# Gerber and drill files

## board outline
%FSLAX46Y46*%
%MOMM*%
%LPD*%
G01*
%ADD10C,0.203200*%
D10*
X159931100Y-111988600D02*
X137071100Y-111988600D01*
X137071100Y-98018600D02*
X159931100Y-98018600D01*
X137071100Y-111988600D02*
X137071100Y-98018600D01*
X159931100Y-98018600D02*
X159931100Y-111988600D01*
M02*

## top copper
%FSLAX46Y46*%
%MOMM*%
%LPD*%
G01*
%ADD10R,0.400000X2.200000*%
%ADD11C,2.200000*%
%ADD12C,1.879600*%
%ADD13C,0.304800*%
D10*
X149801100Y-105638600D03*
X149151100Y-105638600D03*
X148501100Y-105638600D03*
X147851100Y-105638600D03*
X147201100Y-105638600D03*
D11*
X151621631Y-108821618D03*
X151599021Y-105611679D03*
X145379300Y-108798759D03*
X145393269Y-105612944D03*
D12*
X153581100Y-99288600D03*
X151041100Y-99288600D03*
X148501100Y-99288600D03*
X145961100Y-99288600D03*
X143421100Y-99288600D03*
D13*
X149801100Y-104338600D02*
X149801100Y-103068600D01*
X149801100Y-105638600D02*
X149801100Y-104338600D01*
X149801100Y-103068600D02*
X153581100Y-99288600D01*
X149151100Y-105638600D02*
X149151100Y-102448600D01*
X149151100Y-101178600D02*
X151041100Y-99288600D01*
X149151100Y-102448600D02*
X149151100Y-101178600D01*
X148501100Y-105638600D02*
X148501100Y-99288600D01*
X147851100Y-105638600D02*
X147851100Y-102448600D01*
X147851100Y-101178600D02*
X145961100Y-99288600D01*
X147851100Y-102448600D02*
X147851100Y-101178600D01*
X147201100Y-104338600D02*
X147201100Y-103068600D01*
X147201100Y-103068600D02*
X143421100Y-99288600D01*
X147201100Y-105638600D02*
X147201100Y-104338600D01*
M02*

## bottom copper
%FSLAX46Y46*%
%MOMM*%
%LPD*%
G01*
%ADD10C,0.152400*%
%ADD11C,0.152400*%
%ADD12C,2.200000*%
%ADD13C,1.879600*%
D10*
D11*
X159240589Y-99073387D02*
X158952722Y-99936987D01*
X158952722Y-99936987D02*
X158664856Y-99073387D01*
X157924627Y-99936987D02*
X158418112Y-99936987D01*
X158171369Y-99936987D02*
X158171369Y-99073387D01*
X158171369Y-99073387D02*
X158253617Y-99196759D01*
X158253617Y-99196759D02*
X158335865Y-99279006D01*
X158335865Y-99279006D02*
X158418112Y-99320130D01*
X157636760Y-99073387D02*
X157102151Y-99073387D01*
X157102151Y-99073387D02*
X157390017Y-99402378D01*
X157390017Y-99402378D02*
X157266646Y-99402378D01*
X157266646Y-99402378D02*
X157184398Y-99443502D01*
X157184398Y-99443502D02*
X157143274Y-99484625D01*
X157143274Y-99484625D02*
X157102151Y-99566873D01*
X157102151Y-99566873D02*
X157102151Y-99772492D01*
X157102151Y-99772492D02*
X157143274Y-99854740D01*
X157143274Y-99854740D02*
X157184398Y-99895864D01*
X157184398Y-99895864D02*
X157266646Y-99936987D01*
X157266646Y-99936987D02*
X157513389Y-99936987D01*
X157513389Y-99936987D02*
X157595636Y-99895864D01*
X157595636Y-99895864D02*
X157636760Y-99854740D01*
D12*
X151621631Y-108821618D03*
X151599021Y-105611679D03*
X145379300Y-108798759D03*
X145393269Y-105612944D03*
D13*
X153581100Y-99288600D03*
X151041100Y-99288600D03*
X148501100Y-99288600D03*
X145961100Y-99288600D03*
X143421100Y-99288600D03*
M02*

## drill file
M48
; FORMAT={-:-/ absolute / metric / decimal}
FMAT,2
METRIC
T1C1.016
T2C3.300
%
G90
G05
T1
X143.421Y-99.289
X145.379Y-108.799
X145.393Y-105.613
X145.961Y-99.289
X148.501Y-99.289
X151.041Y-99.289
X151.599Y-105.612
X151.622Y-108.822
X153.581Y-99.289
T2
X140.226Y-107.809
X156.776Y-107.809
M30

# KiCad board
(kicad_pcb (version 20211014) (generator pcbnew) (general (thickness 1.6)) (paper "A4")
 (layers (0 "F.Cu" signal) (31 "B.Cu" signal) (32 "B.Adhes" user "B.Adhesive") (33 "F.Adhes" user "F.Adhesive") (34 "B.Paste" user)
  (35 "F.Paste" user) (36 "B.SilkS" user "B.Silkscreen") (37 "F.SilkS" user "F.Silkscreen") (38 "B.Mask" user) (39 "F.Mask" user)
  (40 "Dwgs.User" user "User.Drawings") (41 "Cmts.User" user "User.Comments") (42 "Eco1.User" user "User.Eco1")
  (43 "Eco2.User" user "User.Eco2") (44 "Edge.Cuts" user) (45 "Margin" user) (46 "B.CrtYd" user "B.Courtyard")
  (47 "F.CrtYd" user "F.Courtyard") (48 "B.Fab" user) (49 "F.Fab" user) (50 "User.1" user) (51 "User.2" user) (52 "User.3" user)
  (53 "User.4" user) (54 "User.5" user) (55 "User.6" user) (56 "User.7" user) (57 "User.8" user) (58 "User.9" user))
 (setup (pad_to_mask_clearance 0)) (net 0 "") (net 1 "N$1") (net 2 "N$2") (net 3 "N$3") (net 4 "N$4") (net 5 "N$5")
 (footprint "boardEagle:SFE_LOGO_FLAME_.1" (layer "F.Cu") (at 156.7561 101.3206)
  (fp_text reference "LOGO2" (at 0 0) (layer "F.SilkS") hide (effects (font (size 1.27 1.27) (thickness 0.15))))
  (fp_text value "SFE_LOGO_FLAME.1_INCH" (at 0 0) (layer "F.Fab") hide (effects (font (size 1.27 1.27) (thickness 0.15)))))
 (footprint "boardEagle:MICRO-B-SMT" (layer "F.Cu") (at 148.5011 105.6386 180)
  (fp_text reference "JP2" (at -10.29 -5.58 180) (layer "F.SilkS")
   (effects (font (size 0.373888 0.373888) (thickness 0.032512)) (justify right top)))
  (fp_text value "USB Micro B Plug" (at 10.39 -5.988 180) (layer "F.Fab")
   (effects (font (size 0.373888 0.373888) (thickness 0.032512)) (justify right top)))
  (pad "" np_thru_hole circle (at -8.275 -2.17 180) (size 3.3 3.3) (drill 3.3) (layers *.Cu *.Mask))
  (pad "" np_thru_hole circle (at 8.275 -2.17 180) (size 3.3 3.3) (drill 3.3) (layers *.Cu *.Mask))
  (pad "1" smd rect (at -1.3 0 270) (size 2.2 0.4) (layers "F.Cu" "F.Paste" "F.Mask") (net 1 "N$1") (solder_mask_margin 0.1016))
  (pad "2" smd rect (at -0.65 0 270) (size 2.2 0.4) (layers "F.Cu" "F.Paste" "F.Mask") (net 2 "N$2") (solder_mask_margin 0.1016))
  (pad "3" smd rect (at 0 0 270) (size 2.2 0.4) (layers "F.Cu" "F.Paste" "F.Mask") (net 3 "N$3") (solder_mask_margin 0.1016))
  (pad "4" smd rect (at 0.65 0 270) (size 2.2 0.4) (layers "F.Cu" "F.Paste" "F.Mask") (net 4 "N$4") (solder_mask_margin 0.1016))
  (pad "5" smd rect (at 1.3 0 270) (size 2.2 0.4) (layers "F.Cu" "F.Paste" "F.Mask") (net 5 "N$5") (solder_mask_margin 0.1016))
  (pad "P$6" thru_hole circle (at -3.120531 -3.183018 270) (size 2.2 2.2) (drill 1.016) (layers *.Cu *.Mask) (solder_mask_margin 0.1016))
  (pad "P$7" thru_hole circle (at -3.097921 0.026921 270) (size 2.2 2.2) (drill 1.016) (layers *.Cu *.Mask) (solder_mask_margin 0.1016))
  (pad "P$8" thru_hole circle (at 3.1218 -3.160159 270) (size 2.2 2.2) (drill 1.016) (layers *.Cu *.Mask) (solder_mask_margin 0.1016))
  (pad "P$9" thru_hole circle (at 3.107831 0.025656 270) (size 2.2 2.2) (drill 1.016) (layers *.Cu *.Mask) (solder_mask_margin 0.1016)))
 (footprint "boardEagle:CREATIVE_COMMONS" (layer "F.Cu") (at 121.707044 124.1806)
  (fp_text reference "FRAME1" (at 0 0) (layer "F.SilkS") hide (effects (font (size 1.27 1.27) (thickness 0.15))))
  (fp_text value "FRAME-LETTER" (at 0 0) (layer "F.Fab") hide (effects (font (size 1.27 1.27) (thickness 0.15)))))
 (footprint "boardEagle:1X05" (layer "F.Cu") (at 153.5811 99.2886 180)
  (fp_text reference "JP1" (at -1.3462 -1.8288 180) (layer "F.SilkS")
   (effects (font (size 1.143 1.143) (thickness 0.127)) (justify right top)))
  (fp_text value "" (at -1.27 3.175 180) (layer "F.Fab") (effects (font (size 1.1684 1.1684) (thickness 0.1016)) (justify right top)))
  (pad "1" thru_hole circle (at 0 0 270) (size 1.8796 1.8796) (drill 1.016) (layers *.Cu *.Mask) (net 1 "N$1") (solder_mask_margin 0.1016))
  (pad "2" thru_hole circle (at 2.54 0 270) (size 1.8796 1.8796) (drill 1.016) (layers *.Cu *.Mask) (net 2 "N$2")
   (solder_mask_margin 0.1016))
  (pad "3" thru_hole circle (at 5.08 0 270) (size 1.8796 1.8796) (drill 1.016) (layers *.Cu *.Mask) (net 3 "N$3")
   (solder_mask_margin 0.1016))
  (pad "4" thru_hole circle (at 7.62 0 270) (size 1.8796 1.8796) (drill 1.016) (layers *.Cu *.Mask) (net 4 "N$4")
   (solder_mask_margin 0.1016))
  (pad "5" thru_hole circle (at 10.16 0 270) (size 1.8796 1.8796) (drill 1.016) (layers *.Cu *.Mask) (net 5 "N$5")
   (solder_mask_margin 0.1016)))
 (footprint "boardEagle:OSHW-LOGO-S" (layer "F.Cu") (at 139.2301 99.9236)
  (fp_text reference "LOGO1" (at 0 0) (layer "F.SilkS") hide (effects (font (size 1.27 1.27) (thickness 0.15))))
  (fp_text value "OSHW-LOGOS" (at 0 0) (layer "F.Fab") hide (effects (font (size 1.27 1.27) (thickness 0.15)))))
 (gr_line (start 159.9311 111.9886) (end 137.0711 111.9886) (layer "Edge.Cuts") (width 0.2032))
 (gr_line (start 137.0711 98.0186) (end 159.9311 98.0186) (layer "Edge.Cuts") (width 0.2032))
 (gr_line (start 137.0711 111.9886) (end 137.0711 98.0186) (layer "Edge.Cuts") (width 0.2032))
 (gr_line (start 159.9311 98.0186) (end 159.9311 111.9886) (layer "Edge.Cuts") (width 0.2032))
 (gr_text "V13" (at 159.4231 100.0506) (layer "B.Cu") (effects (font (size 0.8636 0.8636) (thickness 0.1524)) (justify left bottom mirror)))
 (segment (start 149.8011 104.3386) (end 149.8011 103.0686) (width 0.3048) (layer "F.Cu") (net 1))
 (segment (start 149.8011 105.6386) (end 149.8011 104.3386) (width 0.3048) (layer "F.Cu") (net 1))
 (segment (start 149.8011 103.0686) (end 153.5811 99.2886) (width 0.3048) (layer "F.Cu") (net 1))
 (segment (start 149.1511 105.6386) (end 149.1511 102.4486) (width 0.3048) (layer "F.Cu") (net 2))
 (segment (start 149.1511 101.1786) (end 151.0411 99.2886) (width 0.3048) (layer "F.Cu") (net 2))
 (segment (start 149.1511 102.4486) (end 149.1511 101.1786) (width 0.3048) (layer "F.Cu") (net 2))
 (segment (start 148.5011 105.6386) (end 148.5011 99.2886) (width 0.3048) (layer "F.Cu") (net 3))
 (segment (start 147.8511 105.6386) (end 147.8511 102.4486) (width 0.3048) (layer "F.Cu") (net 4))
 (segment (start 147.8511 101.1786) (end 145.9611 99.2886) (width 0.3048) (layer "F.Cu") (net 4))
 (segment (start 147.8511 102.4486) (end 147.8511 101.1786) (width 0.3048) (layer "F.Cu") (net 4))
 (segment (start 147.2011 104.3386) (end 147.2011 103.0686) (width 0.3048) (layer "F.Cu") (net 5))
 (segment (start 147.2011 103.0686) (end 143.4211 99.2886) (width 0.3048) (layer "F.Cu") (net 5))
 (segment (start 147.2011 105.6386) (end 147.2011 104.3386) (width 0.3048) (layer "F.Cu") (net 5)))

